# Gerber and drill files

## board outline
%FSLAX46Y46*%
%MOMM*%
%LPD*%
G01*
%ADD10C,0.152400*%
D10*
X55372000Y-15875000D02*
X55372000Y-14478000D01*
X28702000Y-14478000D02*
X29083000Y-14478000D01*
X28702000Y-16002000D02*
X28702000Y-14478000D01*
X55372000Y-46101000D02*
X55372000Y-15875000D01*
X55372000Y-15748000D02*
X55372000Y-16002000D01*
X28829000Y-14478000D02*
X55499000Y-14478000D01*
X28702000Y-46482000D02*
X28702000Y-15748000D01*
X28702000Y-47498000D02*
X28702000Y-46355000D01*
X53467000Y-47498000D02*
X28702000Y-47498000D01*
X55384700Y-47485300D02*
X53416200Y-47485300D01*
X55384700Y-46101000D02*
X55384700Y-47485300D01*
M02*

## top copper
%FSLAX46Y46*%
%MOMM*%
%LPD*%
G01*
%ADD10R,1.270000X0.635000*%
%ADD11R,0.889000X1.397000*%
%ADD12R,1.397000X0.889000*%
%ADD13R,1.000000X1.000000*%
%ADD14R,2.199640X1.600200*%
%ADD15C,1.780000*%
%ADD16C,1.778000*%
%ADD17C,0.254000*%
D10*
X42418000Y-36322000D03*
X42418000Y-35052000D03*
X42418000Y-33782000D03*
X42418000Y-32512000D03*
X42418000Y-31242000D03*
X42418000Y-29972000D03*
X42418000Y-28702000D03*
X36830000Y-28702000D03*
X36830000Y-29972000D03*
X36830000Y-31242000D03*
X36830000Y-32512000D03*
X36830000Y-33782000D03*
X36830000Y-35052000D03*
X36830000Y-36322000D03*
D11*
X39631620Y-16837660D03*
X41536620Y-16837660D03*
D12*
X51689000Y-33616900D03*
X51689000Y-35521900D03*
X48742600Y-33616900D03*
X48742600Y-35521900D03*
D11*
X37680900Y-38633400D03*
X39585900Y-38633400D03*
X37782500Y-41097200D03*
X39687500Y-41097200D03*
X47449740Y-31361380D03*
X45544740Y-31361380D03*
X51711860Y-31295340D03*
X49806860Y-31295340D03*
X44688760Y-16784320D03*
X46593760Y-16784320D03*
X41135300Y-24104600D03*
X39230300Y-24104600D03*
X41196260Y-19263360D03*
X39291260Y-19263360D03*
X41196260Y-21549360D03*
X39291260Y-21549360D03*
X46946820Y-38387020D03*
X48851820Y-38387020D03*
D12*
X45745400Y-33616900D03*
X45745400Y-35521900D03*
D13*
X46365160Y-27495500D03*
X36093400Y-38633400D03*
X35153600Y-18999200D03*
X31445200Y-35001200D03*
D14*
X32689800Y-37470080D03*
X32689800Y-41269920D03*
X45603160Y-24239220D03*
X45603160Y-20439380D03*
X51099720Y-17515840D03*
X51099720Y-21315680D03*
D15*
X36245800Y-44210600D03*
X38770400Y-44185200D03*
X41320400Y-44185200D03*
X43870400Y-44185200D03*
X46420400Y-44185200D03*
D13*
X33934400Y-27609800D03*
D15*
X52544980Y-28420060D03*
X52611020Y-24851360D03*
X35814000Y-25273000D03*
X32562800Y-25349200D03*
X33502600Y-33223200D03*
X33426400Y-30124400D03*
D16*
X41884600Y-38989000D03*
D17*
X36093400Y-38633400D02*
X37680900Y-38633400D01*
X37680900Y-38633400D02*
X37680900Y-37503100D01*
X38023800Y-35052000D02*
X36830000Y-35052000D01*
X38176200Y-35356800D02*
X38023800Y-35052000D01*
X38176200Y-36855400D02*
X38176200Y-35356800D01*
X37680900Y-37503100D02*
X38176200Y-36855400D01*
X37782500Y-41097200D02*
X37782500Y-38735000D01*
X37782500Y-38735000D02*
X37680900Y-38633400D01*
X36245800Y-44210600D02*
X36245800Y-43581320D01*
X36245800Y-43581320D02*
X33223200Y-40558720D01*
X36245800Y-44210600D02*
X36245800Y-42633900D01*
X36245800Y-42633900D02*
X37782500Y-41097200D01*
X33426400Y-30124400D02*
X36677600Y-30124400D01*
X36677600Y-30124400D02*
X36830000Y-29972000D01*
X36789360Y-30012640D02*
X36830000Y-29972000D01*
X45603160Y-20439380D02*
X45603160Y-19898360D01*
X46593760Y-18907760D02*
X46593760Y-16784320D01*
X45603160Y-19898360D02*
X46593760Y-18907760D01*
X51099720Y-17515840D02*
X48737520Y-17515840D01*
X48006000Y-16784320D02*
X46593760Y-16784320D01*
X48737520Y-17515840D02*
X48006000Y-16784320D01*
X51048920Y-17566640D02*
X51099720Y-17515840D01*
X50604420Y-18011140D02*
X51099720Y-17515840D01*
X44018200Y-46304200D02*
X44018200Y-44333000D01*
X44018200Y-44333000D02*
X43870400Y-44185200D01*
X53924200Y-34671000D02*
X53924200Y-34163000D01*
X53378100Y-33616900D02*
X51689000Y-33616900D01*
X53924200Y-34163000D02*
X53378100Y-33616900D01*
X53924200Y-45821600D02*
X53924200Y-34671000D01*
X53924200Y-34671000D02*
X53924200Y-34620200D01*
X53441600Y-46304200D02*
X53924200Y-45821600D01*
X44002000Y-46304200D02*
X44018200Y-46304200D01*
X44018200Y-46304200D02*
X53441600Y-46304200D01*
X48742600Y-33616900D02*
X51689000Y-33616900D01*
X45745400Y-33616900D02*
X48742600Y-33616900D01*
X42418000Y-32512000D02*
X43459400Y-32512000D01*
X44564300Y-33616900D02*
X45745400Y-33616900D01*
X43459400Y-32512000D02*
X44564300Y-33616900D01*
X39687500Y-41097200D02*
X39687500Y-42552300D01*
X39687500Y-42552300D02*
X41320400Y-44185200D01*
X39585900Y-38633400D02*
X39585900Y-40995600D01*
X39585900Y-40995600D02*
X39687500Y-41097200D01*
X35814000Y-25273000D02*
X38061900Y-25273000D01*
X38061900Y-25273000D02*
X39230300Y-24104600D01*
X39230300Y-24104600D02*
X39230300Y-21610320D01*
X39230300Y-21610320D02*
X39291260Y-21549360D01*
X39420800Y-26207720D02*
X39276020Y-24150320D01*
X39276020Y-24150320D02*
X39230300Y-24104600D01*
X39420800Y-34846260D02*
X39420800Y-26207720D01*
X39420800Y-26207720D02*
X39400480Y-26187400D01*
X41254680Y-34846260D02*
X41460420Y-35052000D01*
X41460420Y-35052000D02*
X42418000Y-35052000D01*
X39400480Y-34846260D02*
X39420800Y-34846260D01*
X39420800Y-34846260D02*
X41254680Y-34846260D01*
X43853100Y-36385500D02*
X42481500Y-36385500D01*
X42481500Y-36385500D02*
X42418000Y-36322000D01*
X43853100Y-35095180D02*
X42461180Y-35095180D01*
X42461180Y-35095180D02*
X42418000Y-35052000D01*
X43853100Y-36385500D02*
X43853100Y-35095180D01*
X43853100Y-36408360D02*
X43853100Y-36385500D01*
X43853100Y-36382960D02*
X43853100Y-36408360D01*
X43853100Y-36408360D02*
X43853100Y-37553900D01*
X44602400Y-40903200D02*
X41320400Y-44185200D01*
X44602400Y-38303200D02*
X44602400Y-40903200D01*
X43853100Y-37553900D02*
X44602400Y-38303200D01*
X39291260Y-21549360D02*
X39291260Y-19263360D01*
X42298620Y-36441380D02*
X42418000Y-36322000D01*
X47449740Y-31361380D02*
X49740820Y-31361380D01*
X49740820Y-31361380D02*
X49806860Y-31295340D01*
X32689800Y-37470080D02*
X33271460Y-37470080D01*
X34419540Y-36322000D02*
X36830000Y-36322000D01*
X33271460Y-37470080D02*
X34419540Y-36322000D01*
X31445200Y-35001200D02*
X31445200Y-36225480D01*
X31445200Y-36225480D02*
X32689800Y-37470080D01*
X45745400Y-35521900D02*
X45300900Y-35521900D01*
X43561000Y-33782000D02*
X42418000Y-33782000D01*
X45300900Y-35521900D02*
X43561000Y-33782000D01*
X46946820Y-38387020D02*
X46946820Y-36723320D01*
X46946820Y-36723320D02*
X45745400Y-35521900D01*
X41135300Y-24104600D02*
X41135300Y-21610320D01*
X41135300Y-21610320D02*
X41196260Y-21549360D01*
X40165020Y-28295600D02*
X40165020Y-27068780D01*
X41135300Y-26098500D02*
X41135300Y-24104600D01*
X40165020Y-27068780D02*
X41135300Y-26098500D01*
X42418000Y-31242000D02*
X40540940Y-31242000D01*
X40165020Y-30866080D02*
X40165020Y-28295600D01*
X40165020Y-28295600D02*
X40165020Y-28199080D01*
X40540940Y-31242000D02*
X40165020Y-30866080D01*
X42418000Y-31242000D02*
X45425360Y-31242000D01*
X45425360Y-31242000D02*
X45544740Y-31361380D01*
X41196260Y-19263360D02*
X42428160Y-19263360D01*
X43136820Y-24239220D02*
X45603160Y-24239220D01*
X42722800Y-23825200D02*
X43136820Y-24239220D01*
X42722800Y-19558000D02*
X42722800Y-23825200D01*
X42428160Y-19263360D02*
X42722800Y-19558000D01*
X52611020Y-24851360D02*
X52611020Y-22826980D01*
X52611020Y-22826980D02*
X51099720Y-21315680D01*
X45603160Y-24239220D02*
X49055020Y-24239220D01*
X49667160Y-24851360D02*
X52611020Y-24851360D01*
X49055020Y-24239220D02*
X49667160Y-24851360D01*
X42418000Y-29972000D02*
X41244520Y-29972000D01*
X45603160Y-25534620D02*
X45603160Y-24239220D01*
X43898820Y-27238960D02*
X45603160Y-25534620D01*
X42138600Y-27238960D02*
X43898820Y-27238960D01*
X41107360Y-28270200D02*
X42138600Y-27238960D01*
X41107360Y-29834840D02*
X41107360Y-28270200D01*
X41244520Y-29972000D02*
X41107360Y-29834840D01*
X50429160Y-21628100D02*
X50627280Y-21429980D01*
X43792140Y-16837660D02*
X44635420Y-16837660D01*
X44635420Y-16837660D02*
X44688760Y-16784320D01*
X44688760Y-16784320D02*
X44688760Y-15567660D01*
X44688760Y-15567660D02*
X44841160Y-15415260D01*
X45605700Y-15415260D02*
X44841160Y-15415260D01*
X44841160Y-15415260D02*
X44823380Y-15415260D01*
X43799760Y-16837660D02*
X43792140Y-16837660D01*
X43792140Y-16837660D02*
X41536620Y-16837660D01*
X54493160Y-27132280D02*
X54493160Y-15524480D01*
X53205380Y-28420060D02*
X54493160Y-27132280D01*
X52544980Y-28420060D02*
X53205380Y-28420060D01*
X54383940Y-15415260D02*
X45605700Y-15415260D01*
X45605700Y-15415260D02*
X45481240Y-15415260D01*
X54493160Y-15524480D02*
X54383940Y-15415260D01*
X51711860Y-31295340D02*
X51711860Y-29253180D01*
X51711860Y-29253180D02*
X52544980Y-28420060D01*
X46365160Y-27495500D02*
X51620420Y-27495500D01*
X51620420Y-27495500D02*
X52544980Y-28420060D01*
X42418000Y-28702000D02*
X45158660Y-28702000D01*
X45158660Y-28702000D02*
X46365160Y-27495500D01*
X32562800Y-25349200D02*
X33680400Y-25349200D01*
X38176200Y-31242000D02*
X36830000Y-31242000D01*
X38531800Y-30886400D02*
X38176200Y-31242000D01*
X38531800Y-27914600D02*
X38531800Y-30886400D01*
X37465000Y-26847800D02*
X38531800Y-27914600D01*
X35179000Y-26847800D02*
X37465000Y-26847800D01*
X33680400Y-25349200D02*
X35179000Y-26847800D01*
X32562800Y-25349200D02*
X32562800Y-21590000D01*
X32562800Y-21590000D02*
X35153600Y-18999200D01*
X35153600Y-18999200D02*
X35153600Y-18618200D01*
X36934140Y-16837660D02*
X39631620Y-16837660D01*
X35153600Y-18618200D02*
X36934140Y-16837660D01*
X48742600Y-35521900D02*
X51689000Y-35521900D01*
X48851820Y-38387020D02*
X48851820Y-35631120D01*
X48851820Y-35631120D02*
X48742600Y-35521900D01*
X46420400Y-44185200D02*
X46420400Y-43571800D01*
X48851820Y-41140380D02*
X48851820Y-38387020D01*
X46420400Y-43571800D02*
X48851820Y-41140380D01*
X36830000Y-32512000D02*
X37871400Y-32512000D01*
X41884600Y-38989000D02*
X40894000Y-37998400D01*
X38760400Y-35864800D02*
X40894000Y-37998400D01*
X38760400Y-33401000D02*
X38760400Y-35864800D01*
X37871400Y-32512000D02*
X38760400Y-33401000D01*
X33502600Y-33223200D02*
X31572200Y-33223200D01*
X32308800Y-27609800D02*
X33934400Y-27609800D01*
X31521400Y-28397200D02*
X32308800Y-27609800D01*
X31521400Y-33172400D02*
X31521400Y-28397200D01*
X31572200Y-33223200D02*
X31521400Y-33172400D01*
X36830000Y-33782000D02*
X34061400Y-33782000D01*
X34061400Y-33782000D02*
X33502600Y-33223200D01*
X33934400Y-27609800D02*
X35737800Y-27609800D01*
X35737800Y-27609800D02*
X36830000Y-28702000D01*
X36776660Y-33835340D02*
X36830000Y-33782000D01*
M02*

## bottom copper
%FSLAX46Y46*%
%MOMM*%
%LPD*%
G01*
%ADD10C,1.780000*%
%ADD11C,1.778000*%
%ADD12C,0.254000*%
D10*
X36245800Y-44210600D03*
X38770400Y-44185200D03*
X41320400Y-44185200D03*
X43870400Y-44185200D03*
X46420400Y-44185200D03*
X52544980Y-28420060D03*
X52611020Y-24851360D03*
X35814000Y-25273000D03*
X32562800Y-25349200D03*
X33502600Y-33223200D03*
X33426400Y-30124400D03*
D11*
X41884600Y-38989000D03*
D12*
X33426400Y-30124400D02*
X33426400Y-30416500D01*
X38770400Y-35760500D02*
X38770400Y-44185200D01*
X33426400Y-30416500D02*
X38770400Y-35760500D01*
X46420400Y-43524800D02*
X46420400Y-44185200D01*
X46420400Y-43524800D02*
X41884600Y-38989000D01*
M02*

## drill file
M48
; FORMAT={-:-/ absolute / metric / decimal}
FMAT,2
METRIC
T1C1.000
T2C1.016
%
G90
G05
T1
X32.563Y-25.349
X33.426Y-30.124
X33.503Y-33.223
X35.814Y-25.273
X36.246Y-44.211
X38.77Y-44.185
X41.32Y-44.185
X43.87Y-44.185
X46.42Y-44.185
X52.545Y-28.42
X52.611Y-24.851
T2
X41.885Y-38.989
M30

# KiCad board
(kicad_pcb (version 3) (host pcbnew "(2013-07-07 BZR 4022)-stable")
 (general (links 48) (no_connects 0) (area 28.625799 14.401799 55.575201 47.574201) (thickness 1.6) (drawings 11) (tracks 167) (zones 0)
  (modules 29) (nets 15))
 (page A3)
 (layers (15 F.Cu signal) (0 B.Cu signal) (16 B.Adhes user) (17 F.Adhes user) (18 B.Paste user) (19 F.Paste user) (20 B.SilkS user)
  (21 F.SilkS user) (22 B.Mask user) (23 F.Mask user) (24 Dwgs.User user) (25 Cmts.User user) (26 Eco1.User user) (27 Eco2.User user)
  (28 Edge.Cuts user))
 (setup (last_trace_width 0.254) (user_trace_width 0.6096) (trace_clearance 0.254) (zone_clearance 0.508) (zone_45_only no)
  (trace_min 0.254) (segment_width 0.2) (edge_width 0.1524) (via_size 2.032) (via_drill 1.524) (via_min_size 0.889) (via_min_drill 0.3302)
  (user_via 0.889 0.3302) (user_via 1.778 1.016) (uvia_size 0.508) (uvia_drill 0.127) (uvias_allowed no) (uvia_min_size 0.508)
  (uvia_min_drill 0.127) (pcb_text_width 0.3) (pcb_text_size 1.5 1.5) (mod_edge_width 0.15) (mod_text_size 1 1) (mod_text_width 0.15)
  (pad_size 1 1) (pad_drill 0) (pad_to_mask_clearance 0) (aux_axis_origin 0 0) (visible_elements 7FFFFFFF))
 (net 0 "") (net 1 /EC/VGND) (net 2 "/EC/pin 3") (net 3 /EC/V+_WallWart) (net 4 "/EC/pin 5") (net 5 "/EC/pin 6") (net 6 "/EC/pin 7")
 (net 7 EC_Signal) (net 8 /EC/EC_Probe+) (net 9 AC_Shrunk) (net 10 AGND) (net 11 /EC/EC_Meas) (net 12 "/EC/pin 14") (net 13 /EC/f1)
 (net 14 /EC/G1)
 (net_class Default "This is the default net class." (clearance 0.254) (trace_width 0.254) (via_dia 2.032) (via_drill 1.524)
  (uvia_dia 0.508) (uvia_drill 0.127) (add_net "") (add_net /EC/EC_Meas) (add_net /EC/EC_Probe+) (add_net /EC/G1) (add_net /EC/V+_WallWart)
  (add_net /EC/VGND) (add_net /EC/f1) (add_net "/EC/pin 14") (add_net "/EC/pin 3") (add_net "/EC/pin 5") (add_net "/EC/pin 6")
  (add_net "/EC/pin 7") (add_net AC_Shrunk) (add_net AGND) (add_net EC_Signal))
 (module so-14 (layer F.Cu) (at 39.624 32.512 90)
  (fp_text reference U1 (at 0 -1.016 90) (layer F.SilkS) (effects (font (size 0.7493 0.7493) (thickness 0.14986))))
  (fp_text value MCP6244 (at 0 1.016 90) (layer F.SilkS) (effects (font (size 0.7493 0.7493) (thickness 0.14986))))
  (pad 1 smd rect (at -3.81 2.794 90) (size 0.635 1.27) (layers F.Cu F.Paste F.Mask) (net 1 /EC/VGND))
  (pad 2 smd rect (at -2.54 2.794 90) (size 0.635 1.27) (layers F.Cu F.Paste F.Mask) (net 1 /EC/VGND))
  (pad 3 smd rect (at -1.27 2.794 90) (size 0.635 1.27) (layers F.Cu F.Paste F.Mask) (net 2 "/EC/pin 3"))
  (pad 4 smd rect (at 0 2.794 90) (size 0.635 1.27) (layers F.Cu F.Paste F.Mask) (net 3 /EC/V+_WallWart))
  (pad 5 smd rect (at 1.27 2.794 90) (size 0.635 1.27) (layers F.Cu F.Paste F.Mask) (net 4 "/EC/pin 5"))
  (pad 6 smd rect (at 2.54 2.794 90) (size 0.635 1.27) (layers F.Cu F.Paste F.Mask) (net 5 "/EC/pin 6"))
  (pad 7 smd rect (at 3.81 2.794 90) (size 0.635 1.27) (layers F.Cu F.Paste F.Mask) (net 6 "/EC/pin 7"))
  (pad 8 smd rect (at 3.81 -2.794 90) (size 0.635 1.27) (layers F.Cu F.Paste F.Mask) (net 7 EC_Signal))
  (pad 9 smd rect (at 2.54 -2.794 90) (size 0.635 1.27) (layers F.Cu F.Paste F.Mask) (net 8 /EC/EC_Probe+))
  (pad 10 smd rect (at 1.27 -2.794 90) (size 0.635 1.27) (layers F.Cu F.Paste F.Mask) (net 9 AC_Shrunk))
  (pad 11 smd rect (at 0 -2.794 90) (size 0.635 1.27) (layers F.Cu F.Paste F.Mask) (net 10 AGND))
  (pad 12 smd rect (at -1.27 -2.794 90) (size 0.635 1.27) (layers F.Cu F.Paste F.Mask) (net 7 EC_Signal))
  (pad 13 smd rect (at -2.54 -2.794 90) (size 0.635 1.27) (layers F.Cu F.Paste F.Mask) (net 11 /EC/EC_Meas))
  (pad 14 smd rect (at -3.81 -2.794 90) (size 0.635 1.27) (layers F.Cu F.Paste F.Mask) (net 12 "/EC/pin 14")))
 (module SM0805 (layer F.Cu) (at 40.58412 16.83766)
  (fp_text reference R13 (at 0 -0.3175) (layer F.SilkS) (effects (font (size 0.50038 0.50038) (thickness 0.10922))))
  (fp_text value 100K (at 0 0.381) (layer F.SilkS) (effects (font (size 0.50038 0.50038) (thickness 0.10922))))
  (pad 1 smd rect (at -0.9525 0) (size 0.889 1.397) (layers F.Cu F.Paste F.Mask) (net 9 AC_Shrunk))
  (pad 2 smd rect (at 0.9525 0) (size 0.889 1.397) (layers F.Cu F.Paste F.Mask) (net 6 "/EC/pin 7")))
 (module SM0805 (layer F.Cu) (at 51.689 34.5694 270)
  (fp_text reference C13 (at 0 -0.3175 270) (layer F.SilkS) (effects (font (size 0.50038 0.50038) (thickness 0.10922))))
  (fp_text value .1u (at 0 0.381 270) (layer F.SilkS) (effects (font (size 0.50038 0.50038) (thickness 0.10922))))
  (pad 1 smd rect (at -0.9525 0 270) (size 0.889 1.397) (layers F.Cu F.Paste F.Mask) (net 3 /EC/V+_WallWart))
  (pad 2 smd rect (at 0.9525 0 270) (size 0.889 1.397) (layers F.Cu F.Paste F.Mask) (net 10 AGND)))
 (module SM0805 (layer F.Cu) (at 48.7426 34.5694 270)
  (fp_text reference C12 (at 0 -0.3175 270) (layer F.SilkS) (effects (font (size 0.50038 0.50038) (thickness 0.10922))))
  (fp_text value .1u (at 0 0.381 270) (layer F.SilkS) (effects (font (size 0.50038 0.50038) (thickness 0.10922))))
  (pad 1 smd rect (at -0.9525 0 270) (size 0.889 1.397) (layers F.Cu F.Paste F.Mask) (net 3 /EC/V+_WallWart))
  (pad 2 smd rect (at 0.9525 0 270) (size 0.889 1.397) (layers F.Cu F.Paste F.Mask) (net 10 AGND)))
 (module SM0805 (layer F.Cu) (at 38.6334 38.6334)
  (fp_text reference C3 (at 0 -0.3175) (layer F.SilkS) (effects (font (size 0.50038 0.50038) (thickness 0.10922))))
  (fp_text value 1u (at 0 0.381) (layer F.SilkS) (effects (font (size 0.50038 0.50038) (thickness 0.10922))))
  (pad 1 smd rect (at -0.9525 0) (size 0.889 1.397) (layers F.Cu F.Paste F.Mask) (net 11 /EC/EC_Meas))
  (pad 2 smd rect (at 0.9525 0) (size 0.889 1.397) (layers F.Cu F.Paste F.Mask) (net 1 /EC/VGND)))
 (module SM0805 (layer F.Cu) (at 38.735 41.0972)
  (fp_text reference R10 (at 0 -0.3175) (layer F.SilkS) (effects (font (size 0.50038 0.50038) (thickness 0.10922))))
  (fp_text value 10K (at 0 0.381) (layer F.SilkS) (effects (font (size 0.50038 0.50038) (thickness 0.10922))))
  (pad 1 smd rect (at -0.9525 0) (size 0.889 1.397) (layers F.Cu F.Paste F.Mask) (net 11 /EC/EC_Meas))
  (pad 2 smd rect (at 0.9525 0) (size 0.889 1.397) (layers F.Cu F.Paste F.Mask) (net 1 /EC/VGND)))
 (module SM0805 (layer F.Cu) (at 46.49724 31.36138 180)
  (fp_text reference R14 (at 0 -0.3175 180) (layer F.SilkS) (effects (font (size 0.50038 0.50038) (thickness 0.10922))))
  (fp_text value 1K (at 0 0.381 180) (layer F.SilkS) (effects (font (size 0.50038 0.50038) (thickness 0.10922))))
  (pad 1 smd rect (at -0.9525 0 180) (size 0.889 1.397) (layers F.Cu F.Paste F.Mask) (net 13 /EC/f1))
  (pad 2 smd rect (at 0.9525 0 180) (size 0.889 1.397) (layers F.Cu F.Paste F.Mask) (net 4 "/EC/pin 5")))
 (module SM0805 (layer F.Cu) (at 50.75936 31.29534 180)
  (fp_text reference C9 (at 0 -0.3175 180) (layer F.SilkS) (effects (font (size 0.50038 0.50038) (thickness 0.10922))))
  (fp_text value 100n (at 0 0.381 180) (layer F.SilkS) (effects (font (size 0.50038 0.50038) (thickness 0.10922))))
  (pad 1 smd rect (at -0.9525 0 180) (size 0.889 1.397) (layers F.Cu F.Paste F.Mask) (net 6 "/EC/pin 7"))
  (pad 2 smd rect (at 0.9525 0 180) (size 0.889 1.397) (layers F.Cu F.Paste F.Mask) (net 13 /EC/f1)))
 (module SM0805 (layer F.Cu) (at 45.64126 16.78432)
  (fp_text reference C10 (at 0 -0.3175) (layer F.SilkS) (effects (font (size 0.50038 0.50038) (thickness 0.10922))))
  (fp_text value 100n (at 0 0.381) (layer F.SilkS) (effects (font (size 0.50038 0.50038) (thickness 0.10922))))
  (pad 1 smd rect (at -0.9525 0) (size 0.889 1.397) (layers F.Cu F.Paste F.Mask) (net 6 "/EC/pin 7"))
  (pad 2 smd rect (at 0.9525 0) (size 0.889 1.397) (layers F.Cu F.Paste F.Mask) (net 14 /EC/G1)))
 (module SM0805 (layer F.Cu) (at 40.1828 24.1046 180)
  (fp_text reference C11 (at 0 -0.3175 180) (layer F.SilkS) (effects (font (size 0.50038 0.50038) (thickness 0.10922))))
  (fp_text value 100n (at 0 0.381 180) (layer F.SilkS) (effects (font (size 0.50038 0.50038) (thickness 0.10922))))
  (pad 1 smd rect (at -0.9525 0 180) (size 0.889 1.397) (layers F.Cu F.Paste F.Mask) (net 4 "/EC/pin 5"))
  (pad 2 smd rect (at 0.9525 0 180) (size 0.889 1.397) (layers F.Cu F.Paste F.Mask) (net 1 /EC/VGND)))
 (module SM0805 (layer F.Cu) (at 40.24376 19.26336 180)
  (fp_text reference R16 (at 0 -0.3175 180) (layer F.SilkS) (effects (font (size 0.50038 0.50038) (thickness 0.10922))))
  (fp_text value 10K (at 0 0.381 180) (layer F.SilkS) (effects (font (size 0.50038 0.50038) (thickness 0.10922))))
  (pad 1 smd rect (at -0.9525 0 180) (size 0.889 1.397) (layers F.Cu F.Paste F.Mask) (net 5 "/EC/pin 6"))
  (pad 2 smd rect (at 0.9525 0 180) (size 0.889 1.397) (layers F.Cu F.Paste F.Mask) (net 1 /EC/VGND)))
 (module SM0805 (layer F.Cu) (at 40.24376 21.54936 180)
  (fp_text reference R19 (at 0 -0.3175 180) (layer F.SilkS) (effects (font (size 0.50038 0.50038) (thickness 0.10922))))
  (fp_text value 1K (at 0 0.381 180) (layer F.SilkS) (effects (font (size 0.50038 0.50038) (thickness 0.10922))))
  (pad 1 smd rect (at -0.9525 0 180) (size 0.889 1.397) (layers F.Cu F.Paste F.Mask) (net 4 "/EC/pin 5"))
  (pad 2 smd rect (at 0.9525 0 180) (size 0.889 1.397) (layers F.Cu F.Paste F.Mask) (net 1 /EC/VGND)))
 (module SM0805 (layer F.Cu) (at 47.89932 38.38702)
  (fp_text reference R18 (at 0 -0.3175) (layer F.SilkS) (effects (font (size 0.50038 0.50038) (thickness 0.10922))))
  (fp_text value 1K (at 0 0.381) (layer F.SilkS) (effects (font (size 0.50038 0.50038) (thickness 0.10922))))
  (pad 1 smd rect (at -0.9525 0) (size 0.889 1.397) (layers F.Cu F.Paste F.Mask) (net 2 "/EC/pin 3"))
  (pad 2 smd rect (at 0.9525 0) (size 0.889 1.397) (layers F.Cu F.Paste F.Mask) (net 10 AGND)))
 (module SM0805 (layer F.Cu) (at 45.7454 34.5694 270)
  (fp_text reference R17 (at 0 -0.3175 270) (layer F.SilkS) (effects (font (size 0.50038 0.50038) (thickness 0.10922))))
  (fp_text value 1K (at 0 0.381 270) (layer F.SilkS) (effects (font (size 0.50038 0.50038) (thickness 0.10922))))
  (pad 1 smd rect (at -0.9525 0 270) (size 0.889 1.397) (layers F.Cu F.Paste F.Mask) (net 3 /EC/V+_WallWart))
  (pad 2 smd rect (at 0.9525 0 270) (size 0.889 1.397) (layers F.Cu F.Paste F.Mask) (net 2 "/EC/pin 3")))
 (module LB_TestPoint (layer F.Cu) (at 46.36516 27.4955)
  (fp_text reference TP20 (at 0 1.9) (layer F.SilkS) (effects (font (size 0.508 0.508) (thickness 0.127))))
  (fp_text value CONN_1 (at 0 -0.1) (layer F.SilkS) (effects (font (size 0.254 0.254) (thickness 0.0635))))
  (pad 1 smd rect (at 0 0) (size 1 1) (layers F.Cu F.Paste F.Mask) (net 6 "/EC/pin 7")))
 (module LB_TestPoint (layer F.Cu) (at 36.0934 38.6334 90)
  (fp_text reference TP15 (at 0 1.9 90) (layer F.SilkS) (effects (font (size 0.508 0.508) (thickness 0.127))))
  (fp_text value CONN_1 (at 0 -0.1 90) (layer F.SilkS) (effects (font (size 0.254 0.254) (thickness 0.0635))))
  (pad 1 smd rect (at 0 0 90) (size 1 1) (layers F.Cu F.Paste F.Mask) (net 11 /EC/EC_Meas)))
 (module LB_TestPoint (layer F.Cu) (at 35.1536 18.9992)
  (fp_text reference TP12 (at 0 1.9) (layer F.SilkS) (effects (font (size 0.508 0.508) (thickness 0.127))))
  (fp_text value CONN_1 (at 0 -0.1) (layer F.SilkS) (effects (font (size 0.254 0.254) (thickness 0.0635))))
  (pad 1 smd rect (at 0 0) (size 1 1) (layers F.Cu F.Paste F.Mask) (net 9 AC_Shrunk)))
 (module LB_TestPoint (layer F.Cu) (at 31.4452 35.0012)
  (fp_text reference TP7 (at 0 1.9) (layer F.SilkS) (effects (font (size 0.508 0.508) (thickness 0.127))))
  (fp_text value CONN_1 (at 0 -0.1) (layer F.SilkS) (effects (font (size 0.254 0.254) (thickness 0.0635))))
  (pad 1 smd rect (at 0 0) (size 1 1) (layers F.Cu F.Paste F.Mask) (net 12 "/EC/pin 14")))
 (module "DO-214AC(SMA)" (layer F.Cu) (at 32.6898 39.37 270)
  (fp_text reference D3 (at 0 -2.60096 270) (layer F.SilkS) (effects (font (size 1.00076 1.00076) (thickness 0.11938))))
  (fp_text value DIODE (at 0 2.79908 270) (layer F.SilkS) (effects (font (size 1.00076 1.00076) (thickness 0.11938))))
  (pad 1 smd rect (at -1.89992 0 270) (size 1.6002 2.19964) (layers F.Cu F.Paste F.Mask) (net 12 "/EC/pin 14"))
  (pad 2 smd rect (at 1.89992 0 270) (size 1.6002 2.19964) (layers F.Cu F.Paste F.Mask) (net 11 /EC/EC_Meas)))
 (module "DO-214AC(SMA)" (layer F.Cu) (at 45.60316 22.3393 90)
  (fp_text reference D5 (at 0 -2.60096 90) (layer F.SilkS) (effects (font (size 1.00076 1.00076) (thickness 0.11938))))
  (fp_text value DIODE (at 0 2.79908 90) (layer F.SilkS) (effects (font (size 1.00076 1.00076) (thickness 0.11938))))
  (pad 1 smd rect (at -1.89992 0 90) (size 1.6002 2.19964) (layers F.Cu F.Paste F.Mask) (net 5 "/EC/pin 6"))
  (pad 2 smd rect (at 1.89992 0 90) (size 1.6002 2.19964) (layers F.Cu F.Paste F.Mask) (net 14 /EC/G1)))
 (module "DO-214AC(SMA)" (layer F.Cu) (at 51.09972 19.41576 270)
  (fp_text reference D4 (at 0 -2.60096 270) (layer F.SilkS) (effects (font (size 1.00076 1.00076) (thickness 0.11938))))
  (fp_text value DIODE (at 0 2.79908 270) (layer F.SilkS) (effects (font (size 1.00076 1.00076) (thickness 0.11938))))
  (pad 1 smd rect (at -1.89992 0 270) (size 1.6002 2.19964) (layers F.Cu F.Paste F.Mask) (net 14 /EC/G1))
  (pad 2 smd rect (at 1.89992 0 270) (size 1.6002 2.19964) (layers F.Cu F.Paste F.Mask) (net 5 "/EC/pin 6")))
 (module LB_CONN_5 (layer F.Cu) (at 36.2458 44.1706)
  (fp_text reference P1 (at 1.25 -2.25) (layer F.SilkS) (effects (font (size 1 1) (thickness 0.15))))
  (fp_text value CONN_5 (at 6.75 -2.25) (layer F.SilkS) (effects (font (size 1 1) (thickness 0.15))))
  (pad 1 thru_hole circle (at 0 0.04) (size 1.78 1.78) (drill 1) (layers *.Cu *.Mask F.SilkS) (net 11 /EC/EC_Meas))
  (pad 2 thru_hole circle (at 2.5246 0.0146) (size 1.78 1.78) (drill 1) (layers *.Cu *.Mask F.SilkS) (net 8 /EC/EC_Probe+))
  (pad 3 thru_hole circle (at 5.0746 0.0146) (size 1.78 1.78) (drill 1) (layers *.Cu *.Mask F.SilkS) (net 1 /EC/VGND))
  (pad 4 thru_hole circle (at 7.6246 0.0146) (size 1.78 1.78) (drill 1) (layers *.Cu *.Mask F.SilkS) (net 3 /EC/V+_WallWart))
  (pad 5 thru_hole circle (at 10.1746 0.0146) (size 1.78 1.78) (drill 1) (layers *.Cu *.Mask F.SilkS) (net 10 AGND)))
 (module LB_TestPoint (layer F.Cu) (at 33.9344 27.6098)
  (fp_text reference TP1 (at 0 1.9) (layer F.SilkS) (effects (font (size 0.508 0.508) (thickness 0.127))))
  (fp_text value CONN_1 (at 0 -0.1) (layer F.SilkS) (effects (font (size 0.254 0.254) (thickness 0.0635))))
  (pad 1 smd rect (at 0 0) (size 1 1) (layers F.Cu F.Paste F.Mask) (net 7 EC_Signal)))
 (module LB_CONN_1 (layer F.Cu) (at 52.54498 28.42006)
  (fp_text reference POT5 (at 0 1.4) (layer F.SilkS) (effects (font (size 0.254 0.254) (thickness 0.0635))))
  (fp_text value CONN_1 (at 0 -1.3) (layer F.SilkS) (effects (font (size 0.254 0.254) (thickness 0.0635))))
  (pad 1 thru_hole circle (at 0 0) (size 1.78 1.78) (drill 1) (layers *.Cu *.Mask F.SilkS) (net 6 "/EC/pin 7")))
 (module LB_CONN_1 (layer F.Cu) (at 52.61102 24.85136)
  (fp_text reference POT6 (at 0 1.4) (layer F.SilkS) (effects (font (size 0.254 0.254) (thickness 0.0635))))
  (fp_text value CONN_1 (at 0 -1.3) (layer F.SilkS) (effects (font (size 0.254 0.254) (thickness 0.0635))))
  (pad 1 thru_hole circle (at 0 0) (size 1.78 1.78) (drill 1) (layers *.Cu *.Mask F.SilkS) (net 5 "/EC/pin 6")))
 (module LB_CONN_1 (layer F.Cu) (at 35.814 25.273)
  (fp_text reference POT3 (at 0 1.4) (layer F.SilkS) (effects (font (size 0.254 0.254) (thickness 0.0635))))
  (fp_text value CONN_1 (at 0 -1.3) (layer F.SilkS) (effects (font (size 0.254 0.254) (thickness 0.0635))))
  (pad 1 thru_hole circle (at 0 0) (size 1.78 1.78) (drill 1) (layers *.Cu *.Mask F.SilkS) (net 1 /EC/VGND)))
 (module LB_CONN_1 (layer F.Cu) (at 32.5628 25.3492)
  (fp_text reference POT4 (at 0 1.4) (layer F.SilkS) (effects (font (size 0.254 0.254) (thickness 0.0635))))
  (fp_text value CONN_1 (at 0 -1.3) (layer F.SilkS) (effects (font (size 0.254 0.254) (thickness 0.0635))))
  (pad 1 thru_hole circle (at 0 0) (size 1.78 1.78) (drill 1) (layers *.Cu *.Mask F.SilkS) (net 9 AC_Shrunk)))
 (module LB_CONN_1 (layer F.Cu) (at 33.5026 33.2232)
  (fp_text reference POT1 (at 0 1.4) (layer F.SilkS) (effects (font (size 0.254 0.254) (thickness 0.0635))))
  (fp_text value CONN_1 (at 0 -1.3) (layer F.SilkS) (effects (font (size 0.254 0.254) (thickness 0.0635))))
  (pad 1 thru_hole circle (at 0 0) (size 1.78 1.78) (drill 1) (layers *.Cu *.Mask F.SilkS) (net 7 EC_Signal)))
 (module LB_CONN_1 (layer F.Cu) (at 33.4264 30.1244)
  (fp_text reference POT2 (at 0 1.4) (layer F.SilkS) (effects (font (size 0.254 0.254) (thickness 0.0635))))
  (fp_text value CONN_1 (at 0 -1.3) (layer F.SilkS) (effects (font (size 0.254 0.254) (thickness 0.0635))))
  (pad 1 thru_hole circle (at 0 0) (size 1.78 1.78) (drill 1) (layers *.Cu *.Mask F.SilkS) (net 8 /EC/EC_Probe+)))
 (gr_line (start 55.372 15.875) (end 55.372 14.478) (angle 90) (layer Edge.Cuts) (width 0.1524))
 (gr_line (start 28.702 14.478) (end 29.083 14.478) (angle 90) (layer Edge.Cuts) (width 0.1524))
 (gr_line (start 28.702 16.002) (end 28.702 14.478) (angle 90) (layer Edge.Cuts) (width 0.1524))
 (gr_line (start 55.372 46.101) (end 55.372 15.875) (angle 90) (layer Edge.Cuts) (width 0.1524))
 (gr_line (start 55.372 15.748) (end 55.372 16.002) (angle 90) (layer Edge.Cuts) (width 0.1524))
 (gr_line (start 28.829 14.478) (end 55.499 14.478) (angle 90) (layer Edge.Cuts) (width 0.1524))
 (gr_line (start 28.702 46.482) (end 28.702 15.748) (angle 90) (layer Edge.Cuts) (width 0.1524))
 (gr_line (start 28.702 47.498) (end 28.702 46.355) (angle 90) (layer Edge.Cuts) (width 0.1524))
 (gr_line (start 53.467 47.498) (end 28.702 47.498) (angle 90) (layer Edge.Cuts) (width 0.1524))
 (gr_line (start 55.3847 47.4853) (end 53.4162 47.4853) (angle 90) (layer Edge.Cuts) (width 0.1524))
 (gr_line (start 55.3847 46.101) (end 55.3847 47.4853) (angle 90) (layer Edge.Cuts) (width 0.1524))
 (segment (start 36.0934 38.6334) (end 37.6809 38.6334) (width 0.254) (layer F.Cu) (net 11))
 (segment (start 37.6809 38.6334) (end 37.6809 37.5031) (width 0.254) (layer F.Cu) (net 11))
 (segment (start 38.0238 35.052) (end 36.83 35.052) (width 0.254) (layer F.Cu) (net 11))
 (segment (start 38.1762 35.3568) (end 38.0238 35.052) (width 0.254) (layer F.Cu) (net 11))
 (segment (start 38.1762 36.8554) (end 38.1762 35.3568) (width 0.254) (layer F.Cu) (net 11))
 (segment (start 37.6809 37.5031) (end 38.1762 36.8554) (width 0.254) (layer F.Cu) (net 11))
 (segment (start 37.7825 41.0972) (end 37.7825 38.735) (width 0.254) (layer F.Cu) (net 11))
 (segment (start 37.7825 38.735) (end 37.6809 38.6334) (width 0.254) (layer F.Cu) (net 11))
 (segment (start 36.2458 44.2106) (end 36.2458 43.58132) (width 0.254) (layer F.Cu) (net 11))
 (segment (start 36.2458 43.58132) (end 33.2232 40.55872) (width 0.254) (layer F.Cu) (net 11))
 (segment (start 36.2458 44.2106) (end 36.2458 42.6339) (width 0.254) (layer F.Cu) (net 11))
 (segment (start 36.2458 42.6339) (end 37.7825 41.0972) (width 0.254) (layer F.Cu) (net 11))
 (segment (start 33.4264 30.1244) (end 33.4264 30.4165) (width 0.254) (layer B.Cu) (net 8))
 (segment (start 38.7704 35.7605) (end 38.7704 44.1852) (width 0.254) (layer B.Cu) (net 8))
 (segment (start 33.4264 30.4165) (end 38.7704 35.7605) (width 0.254) (layer B.Cu) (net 8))
 (segment (start 33.4264 30.1244) (end 36.6776 30.1244) (width 0.254) (layer F.Cu) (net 8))
 (segment (start 36.6776 30.1244) (end 36.83 29.972) (width 0.254) (layer F.Cu) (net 8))
 (segment (start 36.78936 30.01264) (end 36.83 29.972) (width 0.254) (layer F.Cu) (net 8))
 (segment (start 45.60316 20.43938) (end 45.60316 19.89836) (width 0.254) (layer F.Cu) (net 14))
 (segment (start 46.59376 18.90776) (end 46.59376 16.78432) (width 0.254) (layer F.Cu) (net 14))
 (segment (start 45.60316 19.89836) (end 46.59376 18.90776) (width 0.254) (layer F.Cu) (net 14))
 (segment (start 51.09972 17.51584) (end 48.73752 17.51584) (width 0.254) (layer F.Cu) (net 14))
 (segment (start 48.006 16.78432) (end 46.59376 16.78432) (width 0.254) (layer F.Cu) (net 14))
 (segment (start 48.73752 17.51584) (end 48.006 16.78432) (width 0.254) (layer F.Cu) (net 14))
 (segment (start 51.04892 17.56664) (end 51.09972 17.51584) (width 0.254) (layer F.Cu) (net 14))
 (segment (start 50.60442 18.01114) (end 51.09972 17.51584) (width 0.254) (layer F.Cu) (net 14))
 (segment (start 44.0182 46.3042) (end 44.0182 44.333) (width 0.254) (layer F.Cu) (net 3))
 (segment (start 44.0182 44.333) (end 43.8704 44.1852) (width 0.254) (layer F.Cu) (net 3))
 (segment (start 53.9242 34.671) (end 53.9242 34.163) (width 0.254) (layer F.Cu) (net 3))
 (segment (start 53.3781 33.6169) (end 51.689 33.6169) (width 0.254) (layer F.Cu) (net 3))
 (segment (start 53.9242 34.163) (end 53.3781 33.6169) (width 0.254) (layer F.Cu) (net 3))
 (segment (start 53.9242 45.8216) (end 53.9242 34.671) (width 0.254) (layer F.Cu) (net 3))
 (segment (start 53.9242 34.671) (end 53.9242 34.6202) (width 0.254) (layer F.Cu) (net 3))
 (segment (start 53.4416 46.3042) (end 53.9242 45.8216) (width 0.254) (layer F.Cu) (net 3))
 (segment (start 44.002 46.3042) (end 44.0182 46.3042) (width 0.254) (layer F.Cu) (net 3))
 (segment (start 44.0182 46.3042) (end 53.4416 46.3042) (width 0.254) (layer F.Cu) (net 3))
 (segment (start 48.7426 33.6169) (end 51.689 33.6169) (width 0.254) (layer F.Cu) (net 3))
 (segment (start 45.7454 33.6169) (end 48.7426 33.6169) (width 0.254) (layer F.Cu) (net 3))
 (segment (start 42.418 32.512) (end 43.4594 32.512) (width 0.254) (layer F.Cu) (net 3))
 (segment (start 44.5643 33.6169) (end 45.7454 33.6169) (width 0.254) (layer F.Cu) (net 3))
 (segment (start 43.4594 32.512) (end 44.5643 33.6169) (width 0.254) (layer F.Cu) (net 3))
 (segment (start 39.6875 41.0972) (end 39.6875 42.5523) (width 0.254) (layer F.Cu) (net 1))
 (segment (start 39.6875 42.5523) (end 41.3204 44.1852) (width 0.254) (layer F.Cu) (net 1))
 (segment (start 39.5859 38.6334) (end 39.5859 40.9956) (width 0.254) (layer F.Cu) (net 1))
 (segment (start 39.5859 40.9956) (end 39.6875 41.0972) (width 0.254) (layer F.Cu) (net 1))
 (segment (start 35.814 25.273) (end 38.0619 25.273) (width 0.254) (layer F.Cu) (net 1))
 (segment (start 38.0619 25.273) (end 39.2303 24.1046) (width 0.254) (layer F.Cu) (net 1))
 (segment (start 39.2303 24.1046) (end 39.2303 21.61032) (width 0.254) (layer F.Cu) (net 1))
 (segment (start 39.2303 21.61032) (end 39.29126 21.54936) (width 0.254) (layer F.Cu) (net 1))
 (segment (start 39.4208 26.20772) (end 39.27602 24.15032) (width 0.254) (layer F.Cu) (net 1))
 (segment (start 39.27602 24.15032) (end 39.2303 24.1046) (width 0.254) (layer F.Cu) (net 1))
 (segment (start 39.4208 34.84626) (end 39.4208 26.20772) (width 0.254) (layer F.Cu) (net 1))
 (segment (start 39.4208 26.20772) (end 39.40048 26.1874) (width 0.254) (layer F.Cu) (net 1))
 (segment (start 41.25468 34.84626) (end 41.46042 35.052) (width 0.254) (layer F.Cu) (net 1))
 (segment (start 41.46042 35.052) (end 42.418 35.052) (width 0.254) (layer F.Cu) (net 1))
 (segment (start 39.40048 34.84626) (end 39.4208 34.84626) (width 0.254) (layer F.Cu) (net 1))
 (segment (start 39.4208 34.84626) (end 41.25468 34.84626) (width 0.254) (layer F.Cu) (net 1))
 (segment (start 43.8531 36.3855) (end 42.4815 36.3855) (width 0.254) (layer F.Cu) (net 1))
 (segment (start 42.4815 36.3855) (end 42.418 36.322) (width 0.254) (layer F.Cu) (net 1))
 (segment (start 43.8531 35.09518) (end 42.46118 35.09518) (width 0.254) (layer F.Cu) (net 1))
 (segment (start 42.46118 35.09518) (end 42.418 35.052) (width 0.254) (layer F.Cu) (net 1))
 (segment (start 43.8531 36.3855) (end 43.8531 35.09518) (width 0.254) (layer F.Cu) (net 1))
 (segment (start 43.8531 36.40836) (end 43.8531 36.3855) (width 0.254) (layer F.Cu) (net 1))
 (segment (start 43.8531 36.38296) (end 43.8531 36.40836) (width 0.254) (layer F.Cu) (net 1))
 (segment (start 43.8531 36.40836) (end 43.8531 37.5539) (width 0.254) (layer F.Cu) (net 1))
 (segment (start 44.6024 40.9032) (end 41.3204 44.1852) (width 0.254) (layer F.Cu) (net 1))
 (segment (start 44.6024 38.3032) (end 44.6024 40.9032) (width 0.254) (layer F.Cu) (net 1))
 (segment (start 43.8531 37.5539) (end 44.6024 38.3032) (width 0.254) (layer F.Cu) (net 1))
 (segment (start 39.29126 21.54936) (end 39.29126 19.26336) (width 0.254) (layer F.Cu) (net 1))
 (segment (start 42.29862 36.44138) (end 42.418 36.322) (width 0.254) (layer F.Cu) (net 1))
 (segment (start 47.44974 31.36138) (end 49.74082 31.36138) (width 0.254) (layer F.Cu) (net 13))
 (segment (start 49.74082 31.36138) (end 49.80686 31.29534) (width 0.254) (layer F.Cu) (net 13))
 (segment (start 32.6898 37.47008) (end 33.27146 37.47008) (width 0.254) (layer F.Cu) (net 12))
 (segment (start 34.41954 36.322) (end 36.83 36.322) (width 0.254) (layer F.Cu) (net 12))
 (segment (start 33.27146 37.47008) (end 34.41954 36.322) (width 0.254) (layer F.Cu) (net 12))
 (segment (start 31.4452 35.0012) (end 31.4452 36.22548) (width 0.254) (layer F.Cu) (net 12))
 (segment (start 31.4452 36.22548) (end 32.6898 37.47008) (width 0.254) (layer F.Cu) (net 12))
 (segment (start 45.7454 35.5219) (end 45.3009 35.5219) (width 0.254) (layer F.Cu) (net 2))
 (segment (start 43.561 33.782) (end 42.418 33.782) (width 0.254) (layer F.Cu) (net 2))
 (segment (start 45.3009 35.5219) (end 43.561 33.782) (width 0.254) (layer F.Cu) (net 2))
 (segment (start 46.94682 38.38702) (end 46.94682 36.72332) (width 0.254) (layer F.Cu) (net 2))
 (segment (start 46.94682 36.72332) (end 45.7454 35.5219) (width 0.254) (layer F.Cu) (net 2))
 (segment (start 41.1353 24.1046) (end 41.1353 21.61032) (width 0.254) (layer F.Cu) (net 4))
 (segment (start 41.1353 21.61032) (end 41.19626 21.54936) (width 0.254) (layer F.Cu) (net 4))
 (segment (start 40.16502 28.2956) (end 40.16502 27.06878) (width 0.254) (layer F.Cu) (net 4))
 (segment (start 41.1353 26.0985) (end 41.1353 24.1046) (width 0.254) (layer F.Cu) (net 4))
 (segment (start 40.16502 27.06878) (end 41.1353 26.0985) (width 0.254) (layer F.Cu) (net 4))
 (segment (start 42.418 31.242) (end 40.54094 31.242) (width 0.254) (layer F.Cu) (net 4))
 (segment (start 40.16502 30.86608) (end 40.16502 28.2956) (width 0.254) (layer F.Cu) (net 4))
 (segment (start 40.16502 28.2956) (end 40.16502 28.19908) (width 0.254) (layer F.Cu) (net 4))
 (segment (start 40.54094 31.242) (end 40.16502 30.86608) (width 0.254) (layer F.Cu) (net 4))
 (segment (start 42.418 31.242) (end 45.42536 31.242) (width 0.254) (layer F.Cu) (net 4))
 (segment (start 45.42536 31.242) (end 45.54474 31.36138) (width 0.254) (layer F.Cu) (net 4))
 (segment (start 41.19626 19.26336) (end 42.42816 19.26336) (width 0.254) (layer F.Cu) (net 5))
 (segment (start 43.13682 24.23922) (end 45.60316 24.23922) (width 0.254) (layer F.Cu) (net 5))
 (segment (start 42.7228 23.8252) (end 43.13682 24.23922) (width 0.254) (layer F.Cu) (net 5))
 (segment (start 42.7228 19.558) (end 42.7228 23.8252) (width 0.254) (layer F.Cu) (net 5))
 (segment (start 42.42816 19.26336) (end 42.7228 19.558) (width 0.254) (layer F.Cu) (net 5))
 (segment (start 52.61102 24.85136) (end 52.61102 22.82698) (width 0.254) (layer F.Cu) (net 5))
 (segment (start 52.61102 22.82698) (end 51.09972 21.31568) (width 0.254) (layer F.Cu) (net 5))
 (segment (start 45.60316 24.23922) (end 49.05502 24.23922) (width 0.254) (layer F.Cu) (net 5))
 (segment (start 49.66716 24.85136) (end 52.61102 24.85136) (width 0.254) (layer F.Cu) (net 5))
 (segment (start 49.05502 24.23922) (end 49.66716 24.85136) (width 0.254) (layer F.Cu) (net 5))
 (segment (start 42.418 29.972) (end 41.24452 29.972) (width 0.254) (layer F.Cu) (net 5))
 (segment (start 45.60316 25.53462) (end 45.60316 24.23922) (width 0.254) (layer F.Cu) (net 5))
 (segment (start 43.89882 27.23896) (end 45.60316 25.53462) (width 0.254) (layer F.Cu) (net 5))
 (segment (start 42.1386 27.23896) (end 43.89882 27.23896) (width 0.254) (layer F.Cu) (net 5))
 (segment (start 41.10736 28.2702) (end 42.1386 27.23896) (width 0.254) (layer F.Cu) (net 5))
 (segment (start 41.10736 29.83484) (end 41.10736 28.2702) (width 0.254) (layer F.Cu) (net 5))
 (segment (start 41.24452 29.972) (end 41.10736 29.83484) (width 0.254) (layer F.Cu) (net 5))
 (segment (start 50.42916 21.6281) (end 50.62728 21.42998) (width 0.254) (layer F.Cu) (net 5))
 (segment (start 43.79214 16.83766) (end 44.63542 16.83766) (width 0.254) (layer F.Cu) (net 6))
 (segment (start 44.63542 16.83766) (end 44.68876 16.78432) (width 0.254) (layer F.Cu) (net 6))
 (segment (start 44.68876 16.78432) (end 44.68876 15.56766) (width 0.254) (layer F.Cu) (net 6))
 (segment (start 44.68876 15.56766) (end 44.84116 15.41526) (width 0.254) (layer F.Cu) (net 6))
 (segment (start 45.6057 15.41526) (end 44.84116 15.41526) (width 0.254) (layer F.Cu) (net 6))
 (segment (start 44.84116 15.41526) (end 44.82338 15.41526) (width 0.254) (layer F.Cu) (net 6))
 (segment (start 43.79976 16.83766) (end 43.79214 16.83766) (width 0.254) (layer F.Cu) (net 6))
 (segment (start 43.79214 16.83766) (end 41.53662 16.83766) (width 0.254) (layer F.Cu) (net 6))
 (segment (start 54.49316 27.13228) (end 54.49316 15.52448) (width 0.254) (layer F.Cu) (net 6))
 (segment (start 53.20538 28.42006) (end 54.49316 27.13228) (width 0.254) (layer F.Cu) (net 6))
 (segment (start 52.54498 28.42006) (end 53.20538 28.42006) (width 0.254) (layer F.Cu) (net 6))
 (segment (start 54.38394 15.41526) (end 45.6057 15.41526) (width 0.254) (layer F.Cu) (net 6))
 (segment (start 45.6057 15.41526) (end 45.48124 15.41526) (width 0.254) (layer F.Cu) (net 6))
 (segment (start 54.49316 15.52448) (end 54.38394 15.41526) (width 0.254) (layer F.Cu) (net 6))
 (segment (start 51.71186 31.29534) (end 51.71186 29.25318) (width 0.254) (layer F.Cu) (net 6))
 (segment (start 51.71186 29.25318) (end 52.54498 28.42006) (width 0.254) (layer F.Cu) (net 6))
 (segment (start 46.36516 27.4955) (end 51.62042 27.4955) (width 0.254) (layer F.Cu) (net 6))
 (segment (start 51.62042 27.4955) (end 52.54498 28.42006) (width 0.254) (layer F.Cu) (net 6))
 (segment (start 42.418 28.702) (end 45.15866 28.702) (width 0.254) (layer F.Cu) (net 6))
 (segment (start 45.15866 28.702) (end 46.36516 27.4955) (width 0.254) (layer F.Cu) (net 6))
 (segment (start 32.5628 25.3492) (end 33.6804 25.3492) (width 0.254) (layer F.Cu) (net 9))
 (segment (start 38.1762 31.242) (end 36.83 31.242) (width 0.254) (layer F.Cu) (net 9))
 (segment (start 38.5318 30.8864) (end 38.1762 31.242) (width 0.254) (layer F.Cu) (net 9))
 (segment (start 38.5318 27.9146) (end 38.5318 30.8864) (width 0.254) (layer F.Cu) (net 9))
 (segment (start 37.465 26.8478) (end 38.5318 27.9146) (width 0.254) (layer F.Cu) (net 9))
 (segment (start 35.179 26.8478) (end 37.465 26.8478) (width 0.254) (layer F.Cu) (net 9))
 (segment (start 33.6804 25.3492) (end 35.179 26.8478) (width 0.254) (layer F.Cu) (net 9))
 (segment (start 32.5628 25.3492) (end 32.5628 21.59) (width 0.254) (layer F.Cu) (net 9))
 (segment (start 32.5628 21.59) (end 35.1536 18.9992) (width 0.254) (layer F.Cu) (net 9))
 (segment (start 35.1536 18.9992) (end 35.1536 18.6182) (width 0.254) (layer F.Cu) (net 9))
 (segment (start 36.93414 16.83766) (end 39.63162 16.83766) (width 0.254) (layer F.Cu) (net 9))
 (segment (start 35.1536 18.6182) (end 36.93414 16.83766) (width 0.254) (layer F.Cu) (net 9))
 (segment (start 48.7426 35.5219) (end 51.689 35.5219) (width 0.254) (layer F.Cu) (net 10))
 (segment (start 48.85182 38.38702) (end 48.85182 35.63112) (width 0.254) (layer F.Cu) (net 10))
 (segment (start 48.85182 35.63112) (end 48.7426 35.5219) (width 0.254) (layer F.Cu) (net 10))
 (segment (start 46.4204 44.1852) (end 46.4204 43.5718) (width 0.254) (layer F.Cu) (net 10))
 (segment (start 48.85182 41.14038) (end 48.85182 38.38702) (width 0.254) (layer F.Cu) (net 10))
 (segment (start 46.4204 43.5718) (end 48.85182 41.14038) (width 0.254) (layer F.Cu) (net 10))
 (segment (start 36.83 32.512) (end 37.8714 32.512) (width 0.254) (layer F.Cu) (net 10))
 (segment (start 46.4204 43.5248) (end 46.4204 44.1852) (width 0.254) (layer B.Cu) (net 10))
 (segment (start 41.8846 38.989) (end 40.894 37.9984) (width 0.254) (layer F.Cu) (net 10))
 (via (at 41.8846 38.989) (size 1.778) (drill 1.016) (layers F.Cu B.Cu) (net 10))
 (segment (start 46.4204 43.5248) (end 41.8846 38.989) (width 0.254) (layer B.Cu) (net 10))
 (segment (start 38.7604 35.8648) (end 40.894 37.9984) (width 0.254) (layer F.Cu) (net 10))
 (segment (start 38.7604 33.401) (end 38.7604 35.8648) (width 0.254) (layer F.Cu) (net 10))
 (segment (start 37.8714 32.512) (end 38.7604 33.401) (width 0.254) (layer F.Cu) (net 10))
 (segment (start 33.5026 33.2232) (end 31.5722 33.2232) (width 0.254) (layer F.Cu) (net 7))
 (segment (start 32.3088 27.6098) (end 33.9344 27.6098) (width 0.254) (layer F.Cu) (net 7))
 (segment (start 31.5214 28.3972) (end 32.3088 27.6098) (width 0.254) (layer F.Cu) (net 7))
 (segment (start 31.5214 33.1724) (end 31.5214 28.3972) (width 0.254) (layer F.Cu) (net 7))
 (segment (start 31.5722 33.2232) (end 31.5214 33.1724) (width 0.254) (layer F.Cu) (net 7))
 (segment (start 36.83 33.782) (end 34.0614 33.782) (width 0.254) (layer F.Cu) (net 7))
 (segment (start 34.0614 33.782) (end 33.5026 33.2232) (width 0.254) (layer F.Cu) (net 7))
 (segment (start 33.9344 27.6098) (end 35.7378 27.6098) (width 0.254) (layer F.Cu) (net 7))
 (segment (start 35.7378 27.6098) (end 36.83 28.702) (width 0.254) (layer F.Cu) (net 7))
 (segment (start 36.77666 33.83534) (end 36.83 33.782) (width 0.254) (layer F.Cu) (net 7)))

